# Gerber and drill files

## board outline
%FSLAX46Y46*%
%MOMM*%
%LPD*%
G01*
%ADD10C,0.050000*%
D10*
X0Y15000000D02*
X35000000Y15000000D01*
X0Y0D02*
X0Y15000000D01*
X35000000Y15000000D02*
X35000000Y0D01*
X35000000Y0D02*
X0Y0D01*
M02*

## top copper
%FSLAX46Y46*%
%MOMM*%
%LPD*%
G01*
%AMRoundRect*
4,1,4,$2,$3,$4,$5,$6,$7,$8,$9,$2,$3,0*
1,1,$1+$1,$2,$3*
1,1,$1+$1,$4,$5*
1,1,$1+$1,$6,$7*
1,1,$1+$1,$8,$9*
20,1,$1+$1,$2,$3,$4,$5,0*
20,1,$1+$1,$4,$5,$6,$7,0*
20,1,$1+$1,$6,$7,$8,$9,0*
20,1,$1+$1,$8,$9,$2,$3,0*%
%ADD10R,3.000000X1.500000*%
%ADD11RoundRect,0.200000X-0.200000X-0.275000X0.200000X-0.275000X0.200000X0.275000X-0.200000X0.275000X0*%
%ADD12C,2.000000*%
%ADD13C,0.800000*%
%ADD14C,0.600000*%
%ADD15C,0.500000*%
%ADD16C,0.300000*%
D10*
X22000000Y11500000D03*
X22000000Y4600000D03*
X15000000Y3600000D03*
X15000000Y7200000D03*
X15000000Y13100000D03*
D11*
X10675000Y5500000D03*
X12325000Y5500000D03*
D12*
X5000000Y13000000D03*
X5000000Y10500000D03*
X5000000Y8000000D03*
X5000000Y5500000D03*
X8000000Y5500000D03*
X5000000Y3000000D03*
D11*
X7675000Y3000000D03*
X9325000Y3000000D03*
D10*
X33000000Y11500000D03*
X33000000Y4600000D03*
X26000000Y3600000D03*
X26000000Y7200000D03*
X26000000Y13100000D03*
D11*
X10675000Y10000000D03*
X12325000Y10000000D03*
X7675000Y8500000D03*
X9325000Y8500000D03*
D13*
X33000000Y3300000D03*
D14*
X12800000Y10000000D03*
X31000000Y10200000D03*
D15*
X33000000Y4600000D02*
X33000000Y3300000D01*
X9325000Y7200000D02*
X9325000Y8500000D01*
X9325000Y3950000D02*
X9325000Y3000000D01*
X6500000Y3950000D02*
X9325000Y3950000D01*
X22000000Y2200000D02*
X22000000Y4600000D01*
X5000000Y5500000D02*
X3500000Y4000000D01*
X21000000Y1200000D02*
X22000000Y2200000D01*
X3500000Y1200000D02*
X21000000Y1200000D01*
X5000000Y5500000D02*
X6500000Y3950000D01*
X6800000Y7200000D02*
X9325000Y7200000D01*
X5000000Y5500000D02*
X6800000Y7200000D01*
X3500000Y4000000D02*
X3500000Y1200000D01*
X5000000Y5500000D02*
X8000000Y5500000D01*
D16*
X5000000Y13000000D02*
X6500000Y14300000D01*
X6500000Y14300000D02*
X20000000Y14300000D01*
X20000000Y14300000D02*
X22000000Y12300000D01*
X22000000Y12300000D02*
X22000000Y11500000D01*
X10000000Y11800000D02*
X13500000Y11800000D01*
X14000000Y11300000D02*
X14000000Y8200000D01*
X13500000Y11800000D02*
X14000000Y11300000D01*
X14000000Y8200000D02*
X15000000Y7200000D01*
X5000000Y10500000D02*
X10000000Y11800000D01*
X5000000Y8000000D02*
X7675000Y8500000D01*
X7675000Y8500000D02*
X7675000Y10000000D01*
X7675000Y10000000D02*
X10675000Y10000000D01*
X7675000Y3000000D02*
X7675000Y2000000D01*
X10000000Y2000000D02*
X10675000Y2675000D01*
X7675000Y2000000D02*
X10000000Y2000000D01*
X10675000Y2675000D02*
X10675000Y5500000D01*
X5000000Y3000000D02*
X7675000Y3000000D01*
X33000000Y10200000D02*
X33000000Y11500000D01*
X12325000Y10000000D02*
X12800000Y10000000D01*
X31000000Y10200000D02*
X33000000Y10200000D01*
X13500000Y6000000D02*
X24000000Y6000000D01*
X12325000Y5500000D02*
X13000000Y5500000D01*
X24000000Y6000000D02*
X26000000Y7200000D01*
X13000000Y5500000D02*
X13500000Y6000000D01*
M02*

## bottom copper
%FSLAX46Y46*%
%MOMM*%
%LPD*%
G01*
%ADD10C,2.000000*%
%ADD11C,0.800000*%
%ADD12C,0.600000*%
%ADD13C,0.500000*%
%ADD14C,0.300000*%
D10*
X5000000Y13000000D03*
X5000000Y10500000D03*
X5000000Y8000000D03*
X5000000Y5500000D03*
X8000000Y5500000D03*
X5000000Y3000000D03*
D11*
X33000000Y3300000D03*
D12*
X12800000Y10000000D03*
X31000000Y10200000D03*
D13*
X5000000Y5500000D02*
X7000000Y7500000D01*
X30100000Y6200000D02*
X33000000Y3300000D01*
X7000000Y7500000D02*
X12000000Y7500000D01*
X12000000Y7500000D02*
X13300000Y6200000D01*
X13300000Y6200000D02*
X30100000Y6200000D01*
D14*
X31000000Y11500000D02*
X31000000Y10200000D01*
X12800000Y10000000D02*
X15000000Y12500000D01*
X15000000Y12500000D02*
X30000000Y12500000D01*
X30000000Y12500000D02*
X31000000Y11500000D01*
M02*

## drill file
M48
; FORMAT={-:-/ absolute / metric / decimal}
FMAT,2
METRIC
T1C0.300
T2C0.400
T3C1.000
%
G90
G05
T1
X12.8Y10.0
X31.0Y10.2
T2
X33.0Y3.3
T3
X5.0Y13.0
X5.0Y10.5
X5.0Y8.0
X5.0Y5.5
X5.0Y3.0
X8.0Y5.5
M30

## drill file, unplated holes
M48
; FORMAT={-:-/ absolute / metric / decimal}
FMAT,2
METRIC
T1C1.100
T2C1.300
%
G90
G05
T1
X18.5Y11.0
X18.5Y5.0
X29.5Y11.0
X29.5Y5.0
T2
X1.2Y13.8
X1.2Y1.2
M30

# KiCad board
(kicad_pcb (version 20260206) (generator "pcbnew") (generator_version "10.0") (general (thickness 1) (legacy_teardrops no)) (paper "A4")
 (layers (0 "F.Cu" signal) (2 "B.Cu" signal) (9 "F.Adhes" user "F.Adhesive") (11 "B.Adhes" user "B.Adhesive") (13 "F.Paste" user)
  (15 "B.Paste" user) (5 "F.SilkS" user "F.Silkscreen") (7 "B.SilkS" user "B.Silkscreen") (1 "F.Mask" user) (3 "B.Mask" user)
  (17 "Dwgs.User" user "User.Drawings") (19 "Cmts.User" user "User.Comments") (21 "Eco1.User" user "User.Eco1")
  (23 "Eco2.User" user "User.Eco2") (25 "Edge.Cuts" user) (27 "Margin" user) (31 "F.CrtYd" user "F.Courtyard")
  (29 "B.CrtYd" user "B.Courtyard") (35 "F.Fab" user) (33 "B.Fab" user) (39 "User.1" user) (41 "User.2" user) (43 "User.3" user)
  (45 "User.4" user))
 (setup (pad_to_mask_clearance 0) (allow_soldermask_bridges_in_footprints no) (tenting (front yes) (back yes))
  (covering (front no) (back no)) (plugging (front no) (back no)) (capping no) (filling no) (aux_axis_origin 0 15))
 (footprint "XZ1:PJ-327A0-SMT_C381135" (layer "F.Cu") (at 18.5 7 90)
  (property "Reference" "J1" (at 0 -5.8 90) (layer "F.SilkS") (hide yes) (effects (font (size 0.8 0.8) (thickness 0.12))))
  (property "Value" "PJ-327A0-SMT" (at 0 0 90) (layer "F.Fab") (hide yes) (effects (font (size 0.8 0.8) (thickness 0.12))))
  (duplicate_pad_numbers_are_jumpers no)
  (pad "" np_thru_hole circle (at -3 0 90) (size 1.1 1.1) (drill 1.1) (layers "*.Cu" "*.Mask"))
  (pad "" np_thru_hole circle (at 3 0 90) (size 1.1 1.1) (drill 1.1) (layers "*.Cu" "*.Mask"))
  (pad "2" smd rect (at 3.5 3.5 90) (size 1.5 3) (layers "F.Cu" "F.Mask" "F.Paste") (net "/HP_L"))
  (pad "3" smd rect (at -3.4 3.5 90) (size 1.5 3) (layers "F.Cu" "F.Mask" "F.Paste") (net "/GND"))
  (pad "4" smd rect (at -4.4 -3.5 90) (size 1.5 3) (layers "F.Cu" "F.Mask" "F.Paste") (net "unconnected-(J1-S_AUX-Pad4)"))
  (pad "5" smd rect (at -0.8 -3.5 90) (size 1.5 3) (layers "F.Cu" "F.Mask" "F.Paste") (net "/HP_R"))
  (pad "6" smd rect (at 5.1 -3.5 90) (size 1.5 3) (layers "F.Cu" "F.Mask" "F.Paste") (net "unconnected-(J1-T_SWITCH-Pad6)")))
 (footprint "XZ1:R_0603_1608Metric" (layer "F.Cu") (at 11.5 9.5)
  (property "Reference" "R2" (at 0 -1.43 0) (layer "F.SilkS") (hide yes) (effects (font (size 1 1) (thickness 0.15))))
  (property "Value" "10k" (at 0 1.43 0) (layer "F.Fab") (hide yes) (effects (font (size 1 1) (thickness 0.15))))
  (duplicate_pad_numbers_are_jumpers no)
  (pad "1" smd roundrect (at -0.825 0) (size 0.8 0.95) (layers "F.Cu" "F.Mask" "F.Paste") (roundrect_rratio 0.25) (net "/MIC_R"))
  (pad "2" smd roundrect (at 0.825 0) (size 0.8 0.95) (layers "F.Cu" "F.Mask" "F.Paste") (roundrect_rratio 0.25) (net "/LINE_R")))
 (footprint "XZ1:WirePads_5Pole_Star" (layer "F.Cu") (at 0 0)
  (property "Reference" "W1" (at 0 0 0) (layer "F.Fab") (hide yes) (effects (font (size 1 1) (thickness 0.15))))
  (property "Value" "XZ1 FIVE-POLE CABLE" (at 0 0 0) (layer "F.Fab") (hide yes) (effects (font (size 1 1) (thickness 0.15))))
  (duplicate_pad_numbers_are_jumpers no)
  (pad "" np_thru_hole circle (at 1.2 1.2) (size 1.3 1.3) (drill 1.3) (layers "*.Cu" "*.Mask"))
  (pad "" np_thru_hole circle (at 1.2 13.8) (size 1.3 1.3) (drill 1.3) (layers "*.Cu" "*.Mask"))
  (pad "1" thru_hole circle (at 5 2) (size 2 2) (drill 1) (layers "*.Cu" "*.Mask") (remove_unused_layers no) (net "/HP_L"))
  (pad "2" thru_hole circle (at 5 4.5) (size 2 2) (drill 1) (layers "*.Cu" "*.Mask") (remove_unused_layers no) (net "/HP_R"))
  (pad "3" thru_hole circle (at 5 7) (size 2 2) (drill 1) (layers "*.Cu" "*.Mask") (remove_unused_layers no) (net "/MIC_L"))
  (pad "4" thru_hole circle (at 5 9.5) (size 2 2) (drill 1) (layers "*.Cu" "*.Mask") (remove_unused_layers no) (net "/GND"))
  (pad "4b" thru_hole circle (at 8 9.5) (size 2 2) (drill 1) (layers "*.Cu" "*.Mask") (remove_unused_layers no) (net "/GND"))
  (pad "5" thru_hole circle (at 5 12) (size 2 2) (drill 1) (layers "*.Cu" "*.Mask") (remove_unused_layers no) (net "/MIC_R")))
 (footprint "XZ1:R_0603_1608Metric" (layer "F.Cu") (at 8.5 12)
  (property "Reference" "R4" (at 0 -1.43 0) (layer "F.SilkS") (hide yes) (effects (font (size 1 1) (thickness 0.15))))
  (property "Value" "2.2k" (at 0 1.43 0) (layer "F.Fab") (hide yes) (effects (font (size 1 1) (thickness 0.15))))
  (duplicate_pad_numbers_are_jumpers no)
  (pad "1" smd roundrect (at -0.825 0) (size 0.8 0.95) (layers "F.Cu" "F.Mask" "F.Paste") (roundrect_rratio 0.25) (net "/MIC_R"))
  (pad "2" smd roundrect (at 0.825 0) (size 0.8 0.95) (layers "F.Cu" "F.Mask" "F.Paste") (roundrect_rratio 0.25) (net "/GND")))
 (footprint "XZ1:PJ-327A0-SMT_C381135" (layer "F.Cu") (at 29.5 7 90)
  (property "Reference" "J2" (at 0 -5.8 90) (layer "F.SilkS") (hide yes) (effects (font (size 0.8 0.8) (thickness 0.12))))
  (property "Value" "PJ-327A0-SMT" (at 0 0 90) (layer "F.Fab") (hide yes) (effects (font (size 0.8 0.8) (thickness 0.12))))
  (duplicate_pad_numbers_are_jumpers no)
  (pad "" np_thru_hole circle (at -3 0 90) (size 1.1 1.1) (drill 1.1) (layers "*.Cu" "*.Mask"))
  (pad "" np_thru_hole circle (at 3 0 90) (size 1.1 1.1) (drill 1.1) (layers "*.Cu" "*.Mask"))
  (pad "2" smd rect (at 3.5 3.5 90) (size 1.5 3) (layers "F.Cu" "F.Mask" "F.Paste") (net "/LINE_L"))
  (pad "3" smd rect (at -3.4 3.5 90) (size 1.5 3) (layers "F.Cu" "F.Mask" "F.Paste") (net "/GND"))
  (pad "4" smd rect (at -4.4 -3.5 90) (size 1.5 3) (layers "F.Cu" "F.Mask" "F.Paste") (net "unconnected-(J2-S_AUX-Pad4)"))
  (pad "5" smd rect (at -0.8 -3.5 90) (size 1.5 3) (layers "F.Cu" "F.Mask" "F.Paste") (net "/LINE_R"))
  (pad "6" smd rect (at 5.1 -3.5 90) (size 1.5 3) (layers "F.Cu" "F.Mask" "F.Paste") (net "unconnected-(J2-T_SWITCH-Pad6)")))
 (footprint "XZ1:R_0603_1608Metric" (layer "F.Cu") (at 11.5 5)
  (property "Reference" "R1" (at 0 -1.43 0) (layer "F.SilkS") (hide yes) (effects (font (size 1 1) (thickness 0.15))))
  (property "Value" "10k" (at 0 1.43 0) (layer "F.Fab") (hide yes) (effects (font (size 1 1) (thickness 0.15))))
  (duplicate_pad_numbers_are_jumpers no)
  (pad "1" smd roundrect (at -0.825 0) (size 0.8 0.95) (layers "F.Cu" "F.Mask" "F.Paste") (roundrect_rratio 0.25) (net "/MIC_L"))
  (pad "2" smd roundrect (at 0.825 0) (size 0.8 0.95) (layers "F.Cu" "F.Mask" "F.Paste") (roundrect_rratio 0.25) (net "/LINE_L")))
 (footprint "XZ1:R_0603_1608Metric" (layer "F.Cu") (at 8.5 6.5)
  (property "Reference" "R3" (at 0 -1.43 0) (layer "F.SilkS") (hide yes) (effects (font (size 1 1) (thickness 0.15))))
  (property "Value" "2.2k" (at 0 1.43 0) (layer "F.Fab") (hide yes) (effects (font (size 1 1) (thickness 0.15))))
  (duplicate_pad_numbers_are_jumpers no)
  (pad "1" smd roundrect (at -0.825 0) (size 0.8 0.95) (layers "F.Cu" "F.Mask" "F.Paste") (roundrect_rratio 0.25) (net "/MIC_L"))
  (pad "2" smd roundrect (at 0.825 0) (size 0.8 0.95) (layers "F.Cu" "F.Mask" "F.Paste") (roundrect_rratio 0.25) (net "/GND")))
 (gr_line (start 0 0) (end 35 0) (stroke (width 0.05) (type default)) (layer "Edge.Cuts"))
 (gr_line (start 0 15) (end 0 0) (stroke (width 0.05) (type default)) (layer "Edge.Cuts"))
 (gr_line (start 35 0) (end 35 15) (stroke (width 0.05) (type default)) (layer "Edge.Cuts"))
 (gr_line (start 35 15) (end 0 15) (stroke (width 0.05) (type default)) (layer "Edge.Cuts"))
 (segment (start 33 10.4) (end 33 11.7) (width 0.5) (layer "F.Cu") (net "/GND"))
 (segment (start 9.325 7.8) (end 9.325 6.5) (width 0.5) (layer "F.Cu") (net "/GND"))
 (segment (start 9.325 11.05) (end 9.325 12) (width 0.5) (layer "F.Cu") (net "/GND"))
 (segment (start 6.5 11.05) (end 9.325 11.05) (width 0.5) (layer "F.Cu") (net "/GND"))
 (segment (start 22 12.8) (end 22 10.4) (width 0.5) (layer "F.Cu") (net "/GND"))
 (segment (start 5 9.5) (end 3.5 11) (width 0.5) (layer "F.Cu") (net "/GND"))
 (segment (start 21 13.8) (end 22 12.8) (width 0.5) (layer "F.Cu") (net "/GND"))
 (segment (start 3.5 13.8) (end 21 13.8) (width 0.5) (layer "F.Cu") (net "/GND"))
 (segment (start 5 9.5) (end 6.5 11.05) (width 0.5) (layer "F.Cu") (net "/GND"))
 (segment (start 6.8 7.8) (end 9.325 7.8) (width 0.5) (layer "F.Cu") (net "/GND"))
 (segment (start 5 9.5) (end 6.8 7.8) (width 0.5) (layer "F.Cu") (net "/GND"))
 (segment (start 3.5 11) (end 3.5 13.8) (width 0.5) (layer "F.Cu") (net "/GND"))
 (segment (start 5 9.5) (end 8 9.5) (width 0.5) (layer "F.Cu") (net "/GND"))
 (via (at 33 11.7) (size 0.8) (drill 0.4) (layers "F.Cu" "B.Cu") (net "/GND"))
 (segment (start 5 9.5) (end 7 7.5) (width 0.5) (layer "B.Cu") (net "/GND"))
 (segment (start 30.1 8.8) (end 33 11.7) (width 0.5) (layer "B.Cu") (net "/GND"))
 (segment (start 7 7.5) (end 12 7.5) (width 0.5) (layer "B.Cu") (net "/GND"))
 (segment (start 12 7.5) (end 13.3 8.8) (width 0.5) (layer "B.Cu") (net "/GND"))
 (segment (start 13.3 8.8) (end 30.1 8.8) (width 0.5) (layer "B.Cu") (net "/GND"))
 (segment (start 5 2) (end 6.5 0.7) (width 0.3) (layer "F.Cu") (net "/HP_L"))
 (segment (start 6.5 0.7) (end 20 0.7) (width 0.3) (layer "F.Cu") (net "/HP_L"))
 (segment (start 20 0.7) (end 22 2.7) (width 0.3) (layer "F.Cu") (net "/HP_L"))
 (segment (start 22 2.7) (end 22 3.5) (width 0.3) (layer "F.Cu") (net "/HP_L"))
 (segment (start 10 3.2) (end 13.5 3.2) (width 0.3) (layer "F.Cu") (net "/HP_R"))
 (segment (start 14 3.7) (end 14 6.8) (width 0.3) (layer "F.Cu") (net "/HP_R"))
 (segment (start 13.5 3.2) (end 14 3.7) (width 0.3) (layer "F.Cu") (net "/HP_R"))
 (segment (start 14 6.8) (end 15 7.8) (width 0.3) (layer "F.Cu") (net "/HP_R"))
 (segment (start 5 4.5) (end 10 3.2) (width 0.3) (layer "F.Cu") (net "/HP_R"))
 (segment (start 5 7) (end 7.675 6.5) (width 0.3) (layer "F.Cu") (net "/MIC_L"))
 (segment (start 7.675 6.5) (end 7.675 5) (width 0.3) (layer "F.Cu") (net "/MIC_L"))
 (segment (start 7.675 5) (end 10.675 5) (width 0.3) (layer "F.Cu") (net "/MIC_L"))
 (segment (start 7.675 12) (end 7.675 13) (width 0.3) (layer "F.Cu") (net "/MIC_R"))
 (segment (start 10 13) (end 10.675 12.325) (width 0.3) (layer "F.Cu") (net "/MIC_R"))
 (segment (start 7.675 13) (end 10 13) (width 0.3) (layer "F.Cu") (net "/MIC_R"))
 (segment (start 10.675 12.325) (end 10.675 9.5) (width 0.3) (layer "F.Cu") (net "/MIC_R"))
 (segment (start 5 12) (end 7.675 12) (width 0.3) (layer "F.Cu") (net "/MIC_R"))
 (segment (start 33 4.8) (end 33 3.5) (width 0.3) (layer "F.Cu") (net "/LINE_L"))
 (segment (start 12.325 5) (end 12.8 5) (width 0.3) (layer "F.Cu") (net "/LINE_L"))
 (segment (start 31 4.8) (end 33 4.8) (width 0.3) (layer "F.Cu") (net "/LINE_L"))
 (via (at 12.8 5) (size 0.6) (drill 0.3) (layers "F.Cu" "B.Cu") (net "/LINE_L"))
 (via (at 31 4.8) (size 0.6) (drill 0.3) (layers "F.Cu" "B.Cu") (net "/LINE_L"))
 (segment (start 31 3.5) (end 31 4.8) (width 0.3) (layer "B.Cu") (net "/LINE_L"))
 (segment (start 12.8 5) (end 15 2.5) (width 0.3) (layer "B.Cu") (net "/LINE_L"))
 (segment (start 15 2.5) (end 30 2.5) (width 0.3) (layer "B.Cu") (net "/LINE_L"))
 (segment (start 30 2.5) (end 31 3.5) (width 0.3) (layer "B.Cu") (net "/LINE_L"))
 (segment (start 13.5 9) (end 24 9) (width 0.3) (layer "F.Cu") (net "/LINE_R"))
 (segment (start 12.325 9.5) (end 13 9.5) (width 0.3) (layer "F.Cu") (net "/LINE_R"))
 (segment (start 24 9) (end 26 7.8) (width 0.3) (layer "F.Cu") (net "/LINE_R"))
 (segment (start 13 9.5) (end 13.5 9) (width 0.3) (layer "F.Cu") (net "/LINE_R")))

